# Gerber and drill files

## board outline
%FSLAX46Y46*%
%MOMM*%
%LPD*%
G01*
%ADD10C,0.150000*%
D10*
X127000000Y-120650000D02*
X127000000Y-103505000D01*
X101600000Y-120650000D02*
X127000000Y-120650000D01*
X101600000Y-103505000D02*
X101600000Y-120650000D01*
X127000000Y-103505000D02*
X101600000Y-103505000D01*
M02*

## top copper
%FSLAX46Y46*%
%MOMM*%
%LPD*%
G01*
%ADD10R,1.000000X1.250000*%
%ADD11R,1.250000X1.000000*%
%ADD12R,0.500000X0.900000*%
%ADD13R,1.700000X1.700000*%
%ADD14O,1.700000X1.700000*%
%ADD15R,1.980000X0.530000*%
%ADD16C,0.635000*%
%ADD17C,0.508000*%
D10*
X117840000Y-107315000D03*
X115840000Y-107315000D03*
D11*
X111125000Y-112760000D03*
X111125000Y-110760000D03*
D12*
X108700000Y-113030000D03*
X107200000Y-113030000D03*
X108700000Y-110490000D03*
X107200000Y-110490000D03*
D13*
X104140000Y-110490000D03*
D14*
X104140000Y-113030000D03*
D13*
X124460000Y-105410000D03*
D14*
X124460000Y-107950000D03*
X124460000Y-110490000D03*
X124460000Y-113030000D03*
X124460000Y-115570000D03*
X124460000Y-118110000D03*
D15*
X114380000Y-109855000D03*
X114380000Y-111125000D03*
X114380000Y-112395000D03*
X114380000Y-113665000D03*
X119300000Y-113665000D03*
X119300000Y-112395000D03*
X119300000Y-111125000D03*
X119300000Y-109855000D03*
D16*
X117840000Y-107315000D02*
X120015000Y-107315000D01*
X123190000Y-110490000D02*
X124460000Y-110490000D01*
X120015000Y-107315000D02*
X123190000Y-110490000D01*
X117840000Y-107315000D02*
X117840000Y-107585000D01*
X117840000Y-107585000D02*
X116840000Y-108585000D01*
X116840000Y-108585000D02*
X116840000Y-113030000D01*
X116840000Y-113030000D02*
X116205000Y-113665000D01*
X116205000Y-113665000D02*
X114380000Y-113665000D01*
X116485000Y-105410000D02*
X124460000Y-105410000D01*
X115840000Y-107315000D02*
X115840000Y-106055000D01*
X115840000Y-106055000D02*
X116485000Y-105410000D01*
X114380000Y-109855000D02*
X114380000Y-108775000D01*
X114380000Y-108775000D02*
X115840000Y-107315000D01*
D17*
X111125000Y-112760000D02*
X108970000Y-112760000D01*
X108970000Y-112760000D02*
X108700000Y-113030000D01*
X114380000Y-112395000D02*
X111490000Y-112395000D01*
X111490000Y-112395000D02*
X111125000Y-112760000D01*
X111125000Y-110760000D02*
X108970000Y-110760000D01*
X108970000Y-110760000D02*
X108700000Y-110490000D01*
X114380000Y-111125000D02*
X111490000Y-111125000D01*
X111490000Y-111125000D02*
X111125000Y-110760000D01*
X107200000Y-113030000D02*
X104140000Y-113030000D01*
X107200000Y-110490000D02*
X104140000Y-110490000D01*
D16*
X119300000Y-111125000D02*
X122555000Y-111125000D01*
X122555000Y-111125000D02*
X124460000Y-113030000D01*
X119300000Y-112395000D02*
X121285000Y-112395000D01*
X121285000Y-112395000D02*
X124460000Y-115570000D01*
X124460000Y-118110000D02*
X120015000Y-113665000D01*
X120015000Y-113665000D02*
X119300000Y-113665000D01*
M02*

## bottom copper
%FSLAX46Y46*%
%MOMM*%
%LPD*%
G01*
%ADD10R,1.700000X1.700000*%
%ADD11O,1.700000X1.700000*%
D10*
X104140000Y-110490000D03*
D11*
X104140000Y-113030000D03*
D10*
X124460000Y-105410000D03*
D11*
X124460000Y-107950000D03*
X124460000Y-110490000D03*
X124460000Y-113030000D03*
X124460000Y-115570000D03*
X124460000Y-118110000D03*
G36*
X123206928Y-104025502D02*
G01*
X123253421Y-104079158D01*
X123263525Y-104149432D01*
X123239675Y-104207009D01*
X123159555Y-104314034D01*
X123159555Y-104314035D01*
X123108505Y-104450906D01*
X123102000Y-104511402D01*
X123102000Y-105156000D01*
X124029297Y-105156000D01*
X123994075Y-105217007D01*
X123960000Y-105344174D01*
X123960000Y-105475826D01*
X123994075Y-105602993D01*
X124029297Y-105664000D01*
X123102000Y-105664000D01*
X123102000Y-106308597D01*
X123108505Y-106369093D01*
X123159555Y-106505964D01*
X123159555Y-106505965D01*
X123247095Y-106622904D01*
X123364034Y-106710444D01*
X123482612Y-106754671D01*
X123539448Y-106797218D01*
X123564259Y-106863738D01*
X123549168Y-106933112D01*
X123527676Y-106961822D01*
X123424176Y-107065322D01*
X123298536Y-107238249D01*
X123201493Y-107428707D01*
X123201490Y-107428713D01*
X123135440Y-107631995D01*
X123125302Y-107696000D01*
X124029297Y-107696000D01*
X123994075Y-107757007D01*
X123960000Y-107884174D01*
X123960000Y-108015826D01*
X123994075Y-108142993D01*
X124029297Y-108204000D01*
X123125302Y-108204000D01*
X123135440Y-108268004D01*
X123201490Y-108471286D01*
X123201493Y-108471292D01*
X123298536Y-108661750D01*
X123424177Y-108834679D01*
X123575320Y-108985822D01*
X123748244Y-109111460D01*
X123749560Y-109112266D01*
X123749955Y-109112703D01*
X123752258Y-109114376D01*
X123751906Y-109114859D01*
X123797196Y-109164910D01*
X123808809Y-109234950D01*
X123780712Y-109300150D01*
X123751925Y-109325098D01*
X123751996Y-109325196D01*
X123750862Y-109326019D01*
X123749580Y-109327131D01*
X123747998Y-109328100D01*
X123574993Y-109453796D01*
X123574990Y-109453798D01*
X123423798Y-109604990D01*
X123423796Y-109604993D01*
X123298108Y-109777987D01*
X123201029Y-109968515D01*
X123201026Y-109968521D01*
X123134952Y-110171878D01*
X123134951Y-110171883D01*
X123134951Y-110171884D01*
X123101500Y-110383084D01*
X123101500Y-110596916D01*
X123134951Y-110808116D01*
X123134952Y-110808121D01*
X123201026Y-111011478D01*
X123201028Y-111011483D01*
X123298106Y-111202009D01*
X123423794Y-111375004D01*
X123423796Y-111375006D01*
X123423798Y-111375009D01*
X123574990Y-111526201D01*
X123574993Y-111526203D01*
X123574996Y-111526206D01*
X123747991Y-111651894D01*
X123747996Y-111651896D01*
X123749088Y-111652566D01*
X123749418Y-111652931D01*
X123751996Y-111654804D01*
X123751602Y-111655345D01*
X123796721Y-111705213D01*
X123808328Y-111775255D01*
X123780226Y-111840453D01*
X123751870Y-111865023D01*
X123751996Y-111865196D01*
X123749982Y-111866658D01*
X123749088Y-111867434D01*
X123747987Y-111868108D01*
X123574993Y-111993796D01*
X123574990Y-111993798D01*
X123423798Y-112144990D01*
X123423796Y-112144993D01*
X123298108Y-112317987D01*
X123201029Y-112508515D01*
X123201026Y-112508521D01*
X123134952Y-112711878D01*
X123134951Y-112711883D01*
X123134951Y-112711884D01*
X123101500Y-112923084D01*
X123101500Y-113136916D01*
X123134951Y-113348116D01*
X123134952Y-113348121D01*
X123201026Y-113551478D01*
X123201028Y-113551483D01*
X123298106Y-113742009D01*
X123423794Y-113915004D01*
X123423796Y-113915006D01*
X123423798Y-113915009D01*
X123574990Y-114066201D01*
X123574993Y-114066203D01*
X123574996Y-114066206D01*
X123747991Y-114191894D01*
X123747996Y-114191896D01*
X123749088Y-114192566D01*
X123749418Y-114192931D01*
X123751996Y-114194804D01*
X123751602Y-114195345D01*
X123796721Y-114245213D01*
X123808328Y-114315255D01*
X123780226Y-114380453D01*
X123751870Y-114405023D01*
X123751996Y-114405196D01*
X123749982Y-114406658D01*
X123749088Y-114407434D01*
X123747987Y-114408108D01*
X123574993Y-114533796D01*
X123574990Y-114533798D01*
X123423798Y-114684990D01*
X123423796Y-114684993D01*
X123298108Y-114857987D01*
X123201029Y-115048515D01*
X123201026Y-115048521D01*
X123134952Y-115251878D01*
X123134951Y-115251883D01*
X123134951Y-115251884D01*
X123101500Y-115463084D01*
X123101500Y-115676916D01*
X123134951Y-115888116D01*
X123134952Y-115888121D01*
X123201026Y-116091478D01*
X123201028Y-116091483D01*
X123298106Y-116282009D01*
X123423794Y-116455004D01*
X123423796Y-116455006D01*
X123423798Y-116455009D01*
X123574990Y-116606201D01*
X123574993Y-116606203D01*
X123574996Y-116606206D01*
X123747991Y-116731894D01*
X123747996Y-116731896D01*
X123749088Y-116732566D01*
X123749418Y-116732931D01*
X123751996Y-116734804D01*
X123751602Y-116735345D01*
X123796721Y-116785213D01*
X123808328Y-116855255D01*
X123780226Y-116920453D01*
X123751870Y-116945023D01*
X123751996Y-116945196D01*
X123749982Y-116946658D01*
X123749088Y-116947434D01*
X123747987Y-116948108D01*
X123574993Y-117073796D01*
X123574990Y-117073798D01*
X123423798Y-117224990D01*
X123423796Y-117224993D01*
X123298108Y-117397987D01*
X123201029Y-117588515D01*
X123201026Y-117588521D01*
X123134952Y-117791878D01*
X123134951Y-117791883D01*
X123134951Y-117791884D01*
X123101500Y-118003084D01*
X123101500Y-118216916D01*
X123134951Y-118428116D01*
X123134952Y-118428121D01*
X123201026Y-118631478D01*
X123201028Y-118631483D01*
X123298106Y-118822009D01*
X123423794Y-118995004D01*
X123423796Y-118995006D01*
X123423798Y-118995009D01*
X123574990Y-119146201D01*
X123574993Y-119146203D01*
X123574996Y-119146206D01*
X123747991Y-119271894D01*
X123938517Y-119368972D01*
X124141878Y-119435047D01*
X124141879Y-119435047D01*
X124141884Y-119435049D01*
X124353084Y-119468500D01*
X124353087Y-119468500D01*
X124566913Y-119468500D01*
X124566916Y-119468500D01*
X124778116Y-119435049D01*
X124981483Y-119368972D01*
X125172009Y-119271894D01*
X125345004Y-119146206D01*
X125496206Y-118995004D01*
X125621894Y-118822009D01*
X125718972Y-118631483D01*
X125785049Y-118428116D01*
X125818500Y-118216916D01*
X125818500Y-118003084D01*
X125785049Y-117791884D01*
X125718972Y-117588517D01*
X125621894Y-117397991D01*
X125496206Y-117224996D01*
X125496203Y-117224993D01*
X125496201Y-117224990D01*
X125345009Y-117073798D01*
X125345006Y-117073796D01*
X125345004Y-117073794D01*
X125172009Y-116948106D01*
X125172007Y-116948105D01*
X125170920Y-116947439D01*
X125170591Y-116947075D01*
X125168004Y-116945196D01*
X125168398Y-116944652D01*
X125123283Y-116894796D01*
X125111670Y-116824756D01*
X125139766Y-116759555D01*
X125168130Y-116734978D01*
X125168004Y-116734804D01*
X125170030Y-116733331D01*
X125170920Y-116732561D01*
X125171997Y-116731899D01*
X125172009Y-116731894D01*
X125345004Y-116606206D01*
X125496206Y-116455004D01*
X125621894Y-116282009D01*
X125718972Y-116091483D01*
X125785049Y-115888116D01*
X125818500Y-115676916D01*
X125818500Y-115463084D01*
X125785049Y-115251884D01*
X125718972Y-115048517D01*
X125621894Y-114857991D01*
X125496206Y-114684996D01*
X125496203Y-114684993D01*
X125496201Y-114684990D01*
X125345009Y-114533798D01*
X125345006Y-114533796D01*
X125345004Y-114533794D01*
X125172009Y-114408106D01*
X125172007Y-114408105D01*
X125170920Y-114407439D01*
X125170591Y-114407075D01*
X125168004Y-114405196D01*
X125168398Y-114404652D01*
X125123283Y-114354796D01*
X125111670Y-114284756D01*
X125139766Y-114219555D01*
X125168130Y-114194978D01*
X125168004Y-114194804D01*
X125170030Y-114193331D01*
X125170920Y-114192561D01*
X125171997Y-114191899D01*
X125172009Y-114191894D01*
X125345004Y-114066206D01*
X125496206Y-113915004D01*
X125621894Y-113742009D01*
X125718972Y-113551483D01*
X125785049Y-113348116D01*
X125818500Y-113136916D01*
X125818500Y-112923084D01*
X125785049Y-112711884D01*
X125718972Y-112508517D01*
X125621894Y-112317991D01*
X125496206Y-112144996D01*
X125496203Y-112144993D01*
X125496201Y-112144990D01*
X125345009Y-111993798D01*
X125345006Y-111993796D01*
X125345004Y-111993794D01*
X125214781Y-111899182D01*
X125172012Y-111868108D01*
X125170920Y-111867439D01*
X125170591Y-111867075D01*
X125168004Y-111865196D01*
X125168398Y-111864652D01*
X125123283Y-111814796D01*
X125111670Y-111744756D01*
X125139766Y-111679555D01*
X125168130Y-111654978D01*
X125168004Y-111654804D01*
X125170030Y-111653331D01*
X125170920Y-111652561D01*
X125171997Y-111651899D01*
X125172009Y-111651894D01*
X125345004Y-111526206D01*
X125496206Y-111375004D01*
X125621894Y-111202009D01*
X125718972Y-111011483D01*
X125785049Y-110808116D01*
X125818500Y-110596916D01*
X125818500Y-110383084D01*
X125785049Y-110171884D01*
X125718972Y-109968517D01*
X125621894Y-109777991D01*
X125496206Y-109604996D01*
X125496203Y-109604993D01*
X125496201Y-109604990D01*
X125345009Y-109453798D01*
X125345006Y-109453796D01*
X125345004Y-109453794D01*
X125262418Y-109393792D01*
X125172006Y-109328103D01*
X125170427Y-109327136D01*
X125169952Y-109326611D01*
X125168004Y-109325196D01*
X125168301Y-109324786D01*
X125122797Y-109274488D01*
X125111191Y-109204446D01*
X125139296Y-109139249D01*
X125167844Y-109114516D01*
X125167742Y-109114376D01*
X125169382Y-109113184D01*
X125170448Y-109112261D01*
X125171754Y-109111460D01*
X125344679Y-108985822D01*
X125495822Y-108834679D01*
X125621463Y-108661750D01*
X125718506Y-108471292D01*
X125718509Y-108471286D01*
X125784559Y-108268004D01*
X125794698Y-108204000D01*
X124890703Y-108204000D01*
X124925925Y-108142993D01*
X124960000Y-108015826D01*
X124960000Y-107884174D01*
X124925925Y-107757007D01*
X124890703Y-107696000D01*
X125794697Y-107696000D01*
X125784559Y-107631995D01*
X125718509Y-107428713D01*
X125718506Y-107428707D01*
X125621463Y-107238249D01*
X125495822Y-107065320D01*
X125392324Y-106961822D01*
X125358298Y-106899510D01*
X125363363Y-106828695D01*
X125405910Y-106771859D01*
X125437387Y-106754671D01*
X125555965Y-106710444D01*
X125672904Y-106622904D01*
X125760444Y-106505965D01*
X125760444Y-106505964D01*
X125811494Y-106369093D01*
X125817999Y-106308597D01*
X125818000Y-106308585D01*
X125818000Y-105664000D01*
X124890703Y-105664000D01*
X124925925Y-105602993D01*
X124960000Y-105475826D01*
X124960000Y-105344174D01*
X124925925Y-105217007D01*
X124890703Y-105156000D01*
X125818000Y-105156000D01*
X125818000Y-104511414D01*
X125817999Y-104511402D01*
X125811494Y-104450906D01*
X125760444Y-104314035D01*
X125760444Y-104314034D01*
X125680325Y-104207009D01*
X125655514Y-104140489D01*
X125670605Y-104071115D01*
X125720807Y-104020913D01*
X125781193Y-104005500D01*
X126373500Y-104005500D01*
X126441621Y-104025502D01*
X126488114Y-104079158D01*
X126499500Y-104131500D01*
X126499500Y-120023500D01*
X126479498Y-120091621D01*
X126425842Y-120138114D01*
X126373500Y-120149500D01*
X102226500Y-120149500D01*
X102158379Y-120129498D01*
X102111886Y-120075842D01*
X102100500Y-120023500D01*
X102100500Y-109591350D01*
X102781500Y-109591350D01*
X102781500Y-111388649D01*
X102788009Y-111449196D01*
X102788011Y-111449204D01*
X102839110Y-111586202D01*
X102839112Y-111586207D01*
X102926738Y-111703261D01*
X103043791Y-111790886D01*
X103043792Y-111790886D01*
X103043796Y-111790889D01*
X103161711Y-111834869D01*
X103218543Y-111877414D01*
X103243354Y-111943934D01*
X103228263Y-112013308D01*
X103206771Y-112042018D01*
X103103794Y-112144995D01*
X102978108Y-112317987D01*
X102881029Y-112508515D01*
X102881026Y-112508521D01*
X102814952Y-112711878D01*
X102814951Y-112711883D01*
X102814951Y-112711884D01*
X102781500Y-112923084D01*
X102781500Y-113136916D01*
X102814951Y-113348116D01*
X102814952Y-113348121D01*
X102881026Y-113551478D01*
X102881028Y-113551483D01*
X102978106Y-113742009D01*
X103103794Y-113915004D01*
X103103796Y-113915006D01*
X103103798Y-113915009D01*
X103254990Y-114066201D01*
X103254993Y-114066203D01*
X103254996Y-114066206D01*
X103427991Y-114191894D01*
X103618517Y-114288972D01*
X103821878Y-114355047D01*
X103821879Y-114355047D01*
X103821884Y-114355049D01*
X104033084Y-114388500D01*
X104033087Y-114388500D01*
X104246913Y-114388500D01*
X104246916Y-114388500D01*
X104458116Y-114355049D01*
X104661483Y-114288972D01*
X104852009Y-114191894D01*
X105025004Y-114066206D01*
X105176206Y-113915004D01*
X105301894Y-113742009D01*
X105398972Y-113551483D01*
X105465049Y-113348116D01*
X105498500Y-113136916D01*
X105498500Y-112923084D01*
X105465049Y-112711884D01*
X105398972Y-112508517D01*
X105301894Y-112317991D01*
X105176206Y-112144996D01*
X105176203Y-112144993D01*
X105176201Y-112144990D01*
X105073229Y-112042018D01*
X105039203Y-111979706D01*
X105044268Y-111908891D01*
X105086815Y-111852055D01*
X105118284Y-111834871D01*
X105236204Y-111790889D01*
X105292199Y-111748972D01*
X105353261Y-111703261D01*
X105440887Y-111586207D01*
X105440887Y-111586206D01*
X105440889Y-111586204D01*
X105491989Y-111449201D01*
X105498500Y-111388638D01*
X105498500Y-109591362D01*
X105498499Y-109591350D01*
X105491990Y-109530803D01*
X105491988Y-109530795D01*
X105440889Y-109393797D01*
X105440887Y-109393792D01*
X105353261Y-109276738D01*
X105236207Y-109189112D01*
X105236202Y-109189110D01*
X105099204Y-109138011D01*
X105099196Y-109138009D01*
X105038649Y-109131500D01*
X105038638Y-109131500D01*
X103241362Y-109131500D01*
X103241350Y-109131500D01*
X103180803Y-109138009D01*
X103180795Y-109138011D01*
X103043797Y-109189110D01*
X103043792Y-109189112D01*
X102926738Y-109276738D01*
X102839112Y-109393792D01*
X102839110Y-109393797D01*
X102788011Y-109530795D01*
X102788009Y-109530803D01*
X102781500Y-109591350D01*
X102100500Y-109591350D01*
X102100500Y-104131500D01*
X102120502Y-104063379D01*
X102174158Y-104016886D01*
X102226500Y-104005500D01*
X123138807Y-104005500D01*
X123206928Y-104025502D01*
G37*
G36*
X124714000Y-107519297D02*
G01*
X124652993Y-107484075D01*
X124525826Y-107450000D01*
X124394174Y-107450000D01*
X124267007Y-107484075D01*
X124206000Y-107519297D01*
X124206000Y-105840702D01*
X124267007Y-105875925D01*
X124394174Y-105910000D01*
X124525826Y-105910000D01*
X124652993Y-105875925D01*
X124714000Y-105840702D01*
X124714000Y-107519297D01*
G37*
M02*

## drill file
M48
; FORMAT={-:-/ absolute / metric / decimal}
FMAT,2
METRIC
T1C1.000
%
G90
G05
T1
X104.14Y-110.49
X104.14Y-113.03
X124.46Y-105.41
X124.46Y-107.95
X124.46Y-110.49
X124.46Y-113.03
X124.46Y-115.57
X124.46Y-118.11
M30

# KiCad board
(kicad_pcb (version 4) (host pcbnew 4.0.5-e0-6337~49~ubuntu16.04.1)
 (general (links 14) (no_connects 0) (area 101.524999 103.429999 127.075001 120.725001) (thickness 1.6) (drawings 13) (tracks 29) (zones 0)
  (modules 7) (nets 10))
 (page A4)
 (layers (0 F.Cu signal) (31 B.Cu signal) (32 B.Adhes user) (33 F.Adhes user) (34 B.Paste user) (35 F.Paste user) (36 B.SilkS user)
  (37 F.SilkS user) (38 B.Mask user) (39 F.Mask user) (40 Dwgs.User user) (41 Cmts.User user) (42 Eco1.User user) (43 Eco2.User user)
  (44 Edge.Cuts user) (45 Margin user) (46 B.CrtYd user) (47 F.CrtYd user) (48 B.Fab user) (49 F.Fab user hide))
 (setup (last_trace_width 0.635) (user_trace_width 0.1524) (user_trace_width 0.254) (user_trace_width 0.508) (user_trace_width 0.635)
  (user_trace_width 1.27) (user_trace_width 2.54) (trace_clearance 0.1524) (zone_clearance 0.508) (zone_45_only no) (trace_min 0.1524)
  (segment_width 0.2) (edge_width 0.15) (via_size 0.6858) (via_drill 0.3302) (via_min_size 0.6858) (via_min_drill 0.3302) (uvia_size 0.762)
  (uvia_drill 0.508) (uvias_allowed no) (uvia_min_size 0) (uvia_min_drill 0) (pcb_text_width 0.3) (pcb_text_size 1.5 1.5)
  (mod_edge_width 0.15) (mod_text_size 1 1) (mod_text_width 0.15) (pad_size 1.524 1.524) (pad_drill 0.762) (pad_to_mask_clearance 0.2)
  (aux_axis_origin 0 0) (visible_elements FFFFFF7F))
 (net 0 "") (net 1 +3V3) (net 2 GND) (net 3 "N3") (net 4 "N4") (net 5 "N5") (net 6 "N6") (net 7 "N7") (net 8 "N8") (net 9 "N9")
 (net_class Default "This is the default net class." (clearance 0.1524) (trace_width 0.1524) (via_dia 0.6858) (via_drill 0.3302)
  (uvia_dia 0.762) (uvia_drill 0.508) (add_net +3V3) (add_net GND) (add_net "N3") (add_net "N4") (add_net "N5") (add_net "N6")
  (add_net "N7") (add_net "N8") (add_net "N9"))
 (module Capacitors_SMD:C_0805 (layer F.Cu) (at 116.84 107.315 180)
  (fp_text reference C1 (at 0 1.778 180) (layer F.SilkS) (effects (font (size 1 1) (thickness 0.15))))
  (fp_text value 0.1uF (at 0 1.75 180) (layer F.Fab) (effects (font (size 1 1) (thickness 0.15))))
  (pad 1 smd rect (at -1 0 180) (size 1 1.25) (layers F.Cu F.Paste F.Mask) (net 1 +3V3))
  (pad 2 smd rect (at 1 0 180) (size 1 1.25) (layers F.Cu F.Paste F.Mask) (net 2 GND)))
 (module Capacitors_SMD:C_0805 (layer F.Cu) (at 111.125 111.76 90)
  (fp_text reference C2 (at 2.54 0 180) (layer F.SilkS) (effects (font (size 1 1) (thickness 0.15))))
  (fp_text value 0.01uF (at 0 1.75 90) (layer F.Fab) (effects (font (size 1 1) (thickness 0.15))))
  (pad 1 smd rect (at -1 0 90) (size 1 1.25) (layers F.Cu F.Paste F.Mask) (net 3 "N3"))
  (pad 2 smd rect (at 1 0 90) (size 1 1.25) (layers F.Cu F.Paste F.Mask) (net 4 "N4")))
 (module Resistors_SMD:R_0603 (layer F.Cu) (at 107.95 113.03 180)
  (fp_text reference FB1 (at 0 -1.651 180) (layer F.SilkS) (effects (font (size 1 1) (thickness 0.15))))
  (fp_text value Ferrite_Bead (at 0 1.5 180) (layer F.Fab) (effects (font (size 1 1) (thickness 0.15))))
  (pad 1 smd rect (at -0.75 0 180) (size 0.5 0.9) (layers F.Cu F.Paste F.Mask) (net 3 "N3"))
  (pad 2 smd rect (at 0.75 0 180) (size 0.5 0.9) (layers F.Cu F.Paste F.Mask) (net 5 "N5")))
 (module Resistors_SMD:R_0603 (layer F.Cu) (at 107.95 110.49 180)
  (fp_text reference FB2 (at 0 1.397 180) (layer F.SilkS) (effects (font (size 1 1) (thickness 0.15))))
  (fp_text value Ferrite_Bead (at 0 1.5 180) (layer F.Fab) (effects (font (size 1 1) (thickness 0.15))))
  (pad 1 smd rect (at -0.75 0 180) (size 0.5 0.9) (layers F.Cu F.Paste F.Mask) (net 4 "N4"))
  (pad 2 smd rect (at 0.75 0 180) (size 0.5 0.9) (layers F.Cu F.Paste F.Mask) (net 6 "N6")))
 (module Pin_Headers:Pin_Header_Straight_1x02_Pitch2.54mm (layer F.Cu) (at 104.14 110.49)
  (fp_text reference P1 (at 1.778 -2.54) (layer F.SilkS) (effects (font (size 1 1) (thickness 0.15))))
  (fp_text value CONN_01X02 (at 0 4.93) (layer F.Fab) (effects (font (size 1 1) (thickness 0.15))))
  (pad 1 thru_hole rect (at 0 0) (size 1.7 1.7) (drill 1) (layers *.Cu *.Mask) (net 6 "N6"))
  (pad 2 thru_hole oval (at 0 2.54) (size 1.7 1.7) (drill 1) (layers *.Cu *.Mask) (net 5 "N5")))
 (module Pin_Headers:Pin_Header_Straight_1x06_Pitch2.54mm (layer F.Cu) (at 124.46 105.41)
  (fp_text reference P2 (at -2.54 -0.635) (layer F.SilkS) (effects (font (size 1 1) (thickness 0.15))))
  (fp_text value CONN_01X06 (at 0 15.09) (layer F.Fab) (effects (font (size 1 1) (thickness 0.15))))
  (pad 1 thru_hole rect (at 0 0) (size 1.7 1.7) (drill 1) (layers *.Cu *.Mask) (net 2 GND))
  (pad 2 thru_hole oval (at 0 2.54) (size 1.7 1.7) (drill 1) (layers *.Cu *.Mask) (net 2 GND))
  (pad 3 thru_hole oval (at 0 5.08) (size 1.7 1.7) (drill 1) (layers *.Cu *.Mask) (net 1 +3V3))
  (pad 4 thru_hole oval (at 0 7.62) (size 1.7 1.7) (drill 1) (layers *.Cu *.Mask) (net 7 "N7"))
  (pad 5 thru_hole oval (at 0 10.16) (size 1.7 1.7) (drill 1) (layers *.Cu *.Mask) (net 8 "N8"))
  (pad 6 thru_hole oval (at 0 12.7) (size 1.7 1.7) (drill 1) (layers *.Cu *.Mask) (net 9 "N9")))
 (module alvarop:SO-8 (layer F.Cu) (at 116.84 111.76)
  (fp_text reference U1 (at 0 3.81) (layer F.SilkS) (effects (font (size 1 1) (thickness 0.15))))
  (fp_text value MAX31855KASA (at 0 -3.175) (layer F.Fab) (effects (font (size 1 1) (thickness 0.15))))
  (pad 1 smd rect (at -2.46 -1.905) (size 1.98 0.53) (layers F.Cu F.Paste F.Mask) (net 2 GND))
  (pad 2 smd rect (at -2.46 -0.635) (size 1.98 0.53) (layers F.Cu F.Paste F.Mask) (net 4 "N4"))
  (pad 3 smd rect (at -2.46 0.635) (size 1.98 0.53) (layers F.Cu F.Paste F.Mask) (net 3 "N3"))
  (pad 4 smd rect (at -2.46 1.905) (size 1.98 0.53) (layers F.Cu F.Paste F.Mask) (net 1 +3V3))
  (pad 5 smd rect (at 2.46 1.905) (size 1.98 0.53) (layers F.Cu F.Paste F.Mask) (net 9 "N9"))
  (pad 6 smd rect (at 2.46 0.635) (size 1.98 0.53) (layers F.Cu F.Paste F.Mask) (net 8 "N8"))
  (pad 7 smd rect (at 2.46 -0.635) (size 1.98 0.53) (layers F.Cu F.Paste F.Mask) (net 7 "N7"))
  (pad 8 smd rect (at 2.46 -1.905) (size 1.98 0.53) (layers F.Cu F.Paste F.Mask)))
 (gr_line (start 127 120.65) (end 127 103.505) (layer Edge.Cuts) (width 0.15))
 (gr_line (start 101.6 120.65) (end 127 120.65) (layer Edge.Cuts) (width 0.15))
 (gr_line (start 101.6 103.505) (end 101.6 120.65) (layer Edge.Cuts) (width 0.15))
 (gr_line (start 127 103.505) (end 101.6 103.505) (layer Edge.Cuts) (width 0.15))
 (segment (start 117.84 107.315) (end 120.015 107.315) (width 0.635) (layer F.Cu) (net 1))
 (segment (start 123.19 110.49) (end 124.46 110.49) (width 0.635) (layer F.Cu) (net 1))
 (segment (start 120.015 107.315) (end 123.19 110.49) (width 0.635) (layer F.Cu) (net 1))
 (segment (start 117.84 107.315) (end 117.84 107.585) (width 0.635) (layer F.Cu) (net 1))
 (segment (start 117.84 107.585) (end 116.84 108.585) (width 0.635) (layer F.Cu) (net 1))
 (segment (start 116.84 108.585) (end 116.84 113.03) (width 0.635) (layer F.Cu) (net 1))
 (segment (start 116.84 113.03) (end 116.205 113.665) (width 0.635) (layer F.Cu) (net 1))
 (segment (start 116.205 113.665) (end 114.38 113.665) (width 0.635) (layer F.Cu) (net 1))
 (segment (start 116.485 105.41) (end 124.46 105.41) (width 0.635) (layer F.Cu) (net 2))
 (segment (start 115.84 107.315) (end 115.84 106.055) (width 0.635) (layer F.Cu) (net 2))
 (segment (start 115.84 106.055) (end 116.485 105.41) (width 0.635) (layer F.Cu) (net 2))
 (segment (start 114.38 109.855) (end 114.38 108.775) (width 0.635) (layer F.Cu) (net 2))
 (segment (start 114.38 108.775) (end 115.84 107.315) (width 0.635) (layer F.Cu) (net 2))
 (segment (start 111.125 112.76) (end 108.97 112.76) (width 0.508) (layer F.Cu) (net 3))
 (segment (start 108.97 112.76) (end 108.7 113.03) (width 0.508) (layer F.Cu) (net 3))
 (segment (start 114.38 112.395) (end 111.49 112.395) (width 0.508) (layer F.Cu) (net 3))
 (segment (start 111.49 112.395) (end 111.125 112.76) (width 0.508) (layer F.Cu) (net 3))
 (segment (start 111.125 110.76) (end 108.97 110.76) (width 0.508) (layer F.Cu) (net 4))
 (segment (start 108.97 110.76) (end 108.7 110.49) (width 0.508) (layer F.Cu) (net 4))
 (segment (start 114.38 111.125) (end 111.49 111.125) (width 0.508) (layer F.Cu) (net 4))
 (segment (start 111.49 111.125) (end 111.125 110.76) (width 0.508) (layer F.Cu) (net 4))
 (segment (start 107.2 113.03) (end 104.14 113.03) (width 0.508) (layer F.Cu) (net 5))
 (segment (start 107.2 110.49) (end 104.14 110.49) (width 0.508) (layer F.Cu) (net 6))
 (segment (start 119.3 111.125) (end 122.555 111.125) (width 0.635) (layer F.Cu) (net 7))
 (segment (start 122.555 111.125) (end 124.46 113.03) (width 0.635) (layer F.Cu) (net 7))
 (segment (start 119.3 112.395) (end 121.285 112.395) (width 0.635) (layer F.Cu) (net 8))
 (segment (start 121.285 112.395) (end 124.46 115.57) (width 0.635) (layer F.Cu) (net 8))
 (segment (start 124.46 118.11) (end 120.015 113.665) (width 0.635) (layer F.Cu) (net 9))
 (segment (start 120.015 113.665) (end 119.3 113.665) (width 0.635) (layer F.Cu) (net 9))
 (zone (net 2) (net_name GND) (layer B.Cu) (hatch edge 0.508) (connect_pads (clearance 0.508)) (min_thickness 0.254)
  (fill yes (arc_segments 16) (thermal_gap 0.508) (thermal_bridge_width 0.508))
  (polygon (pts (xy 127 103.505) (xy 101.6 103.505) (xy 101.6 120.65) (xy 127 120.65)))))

